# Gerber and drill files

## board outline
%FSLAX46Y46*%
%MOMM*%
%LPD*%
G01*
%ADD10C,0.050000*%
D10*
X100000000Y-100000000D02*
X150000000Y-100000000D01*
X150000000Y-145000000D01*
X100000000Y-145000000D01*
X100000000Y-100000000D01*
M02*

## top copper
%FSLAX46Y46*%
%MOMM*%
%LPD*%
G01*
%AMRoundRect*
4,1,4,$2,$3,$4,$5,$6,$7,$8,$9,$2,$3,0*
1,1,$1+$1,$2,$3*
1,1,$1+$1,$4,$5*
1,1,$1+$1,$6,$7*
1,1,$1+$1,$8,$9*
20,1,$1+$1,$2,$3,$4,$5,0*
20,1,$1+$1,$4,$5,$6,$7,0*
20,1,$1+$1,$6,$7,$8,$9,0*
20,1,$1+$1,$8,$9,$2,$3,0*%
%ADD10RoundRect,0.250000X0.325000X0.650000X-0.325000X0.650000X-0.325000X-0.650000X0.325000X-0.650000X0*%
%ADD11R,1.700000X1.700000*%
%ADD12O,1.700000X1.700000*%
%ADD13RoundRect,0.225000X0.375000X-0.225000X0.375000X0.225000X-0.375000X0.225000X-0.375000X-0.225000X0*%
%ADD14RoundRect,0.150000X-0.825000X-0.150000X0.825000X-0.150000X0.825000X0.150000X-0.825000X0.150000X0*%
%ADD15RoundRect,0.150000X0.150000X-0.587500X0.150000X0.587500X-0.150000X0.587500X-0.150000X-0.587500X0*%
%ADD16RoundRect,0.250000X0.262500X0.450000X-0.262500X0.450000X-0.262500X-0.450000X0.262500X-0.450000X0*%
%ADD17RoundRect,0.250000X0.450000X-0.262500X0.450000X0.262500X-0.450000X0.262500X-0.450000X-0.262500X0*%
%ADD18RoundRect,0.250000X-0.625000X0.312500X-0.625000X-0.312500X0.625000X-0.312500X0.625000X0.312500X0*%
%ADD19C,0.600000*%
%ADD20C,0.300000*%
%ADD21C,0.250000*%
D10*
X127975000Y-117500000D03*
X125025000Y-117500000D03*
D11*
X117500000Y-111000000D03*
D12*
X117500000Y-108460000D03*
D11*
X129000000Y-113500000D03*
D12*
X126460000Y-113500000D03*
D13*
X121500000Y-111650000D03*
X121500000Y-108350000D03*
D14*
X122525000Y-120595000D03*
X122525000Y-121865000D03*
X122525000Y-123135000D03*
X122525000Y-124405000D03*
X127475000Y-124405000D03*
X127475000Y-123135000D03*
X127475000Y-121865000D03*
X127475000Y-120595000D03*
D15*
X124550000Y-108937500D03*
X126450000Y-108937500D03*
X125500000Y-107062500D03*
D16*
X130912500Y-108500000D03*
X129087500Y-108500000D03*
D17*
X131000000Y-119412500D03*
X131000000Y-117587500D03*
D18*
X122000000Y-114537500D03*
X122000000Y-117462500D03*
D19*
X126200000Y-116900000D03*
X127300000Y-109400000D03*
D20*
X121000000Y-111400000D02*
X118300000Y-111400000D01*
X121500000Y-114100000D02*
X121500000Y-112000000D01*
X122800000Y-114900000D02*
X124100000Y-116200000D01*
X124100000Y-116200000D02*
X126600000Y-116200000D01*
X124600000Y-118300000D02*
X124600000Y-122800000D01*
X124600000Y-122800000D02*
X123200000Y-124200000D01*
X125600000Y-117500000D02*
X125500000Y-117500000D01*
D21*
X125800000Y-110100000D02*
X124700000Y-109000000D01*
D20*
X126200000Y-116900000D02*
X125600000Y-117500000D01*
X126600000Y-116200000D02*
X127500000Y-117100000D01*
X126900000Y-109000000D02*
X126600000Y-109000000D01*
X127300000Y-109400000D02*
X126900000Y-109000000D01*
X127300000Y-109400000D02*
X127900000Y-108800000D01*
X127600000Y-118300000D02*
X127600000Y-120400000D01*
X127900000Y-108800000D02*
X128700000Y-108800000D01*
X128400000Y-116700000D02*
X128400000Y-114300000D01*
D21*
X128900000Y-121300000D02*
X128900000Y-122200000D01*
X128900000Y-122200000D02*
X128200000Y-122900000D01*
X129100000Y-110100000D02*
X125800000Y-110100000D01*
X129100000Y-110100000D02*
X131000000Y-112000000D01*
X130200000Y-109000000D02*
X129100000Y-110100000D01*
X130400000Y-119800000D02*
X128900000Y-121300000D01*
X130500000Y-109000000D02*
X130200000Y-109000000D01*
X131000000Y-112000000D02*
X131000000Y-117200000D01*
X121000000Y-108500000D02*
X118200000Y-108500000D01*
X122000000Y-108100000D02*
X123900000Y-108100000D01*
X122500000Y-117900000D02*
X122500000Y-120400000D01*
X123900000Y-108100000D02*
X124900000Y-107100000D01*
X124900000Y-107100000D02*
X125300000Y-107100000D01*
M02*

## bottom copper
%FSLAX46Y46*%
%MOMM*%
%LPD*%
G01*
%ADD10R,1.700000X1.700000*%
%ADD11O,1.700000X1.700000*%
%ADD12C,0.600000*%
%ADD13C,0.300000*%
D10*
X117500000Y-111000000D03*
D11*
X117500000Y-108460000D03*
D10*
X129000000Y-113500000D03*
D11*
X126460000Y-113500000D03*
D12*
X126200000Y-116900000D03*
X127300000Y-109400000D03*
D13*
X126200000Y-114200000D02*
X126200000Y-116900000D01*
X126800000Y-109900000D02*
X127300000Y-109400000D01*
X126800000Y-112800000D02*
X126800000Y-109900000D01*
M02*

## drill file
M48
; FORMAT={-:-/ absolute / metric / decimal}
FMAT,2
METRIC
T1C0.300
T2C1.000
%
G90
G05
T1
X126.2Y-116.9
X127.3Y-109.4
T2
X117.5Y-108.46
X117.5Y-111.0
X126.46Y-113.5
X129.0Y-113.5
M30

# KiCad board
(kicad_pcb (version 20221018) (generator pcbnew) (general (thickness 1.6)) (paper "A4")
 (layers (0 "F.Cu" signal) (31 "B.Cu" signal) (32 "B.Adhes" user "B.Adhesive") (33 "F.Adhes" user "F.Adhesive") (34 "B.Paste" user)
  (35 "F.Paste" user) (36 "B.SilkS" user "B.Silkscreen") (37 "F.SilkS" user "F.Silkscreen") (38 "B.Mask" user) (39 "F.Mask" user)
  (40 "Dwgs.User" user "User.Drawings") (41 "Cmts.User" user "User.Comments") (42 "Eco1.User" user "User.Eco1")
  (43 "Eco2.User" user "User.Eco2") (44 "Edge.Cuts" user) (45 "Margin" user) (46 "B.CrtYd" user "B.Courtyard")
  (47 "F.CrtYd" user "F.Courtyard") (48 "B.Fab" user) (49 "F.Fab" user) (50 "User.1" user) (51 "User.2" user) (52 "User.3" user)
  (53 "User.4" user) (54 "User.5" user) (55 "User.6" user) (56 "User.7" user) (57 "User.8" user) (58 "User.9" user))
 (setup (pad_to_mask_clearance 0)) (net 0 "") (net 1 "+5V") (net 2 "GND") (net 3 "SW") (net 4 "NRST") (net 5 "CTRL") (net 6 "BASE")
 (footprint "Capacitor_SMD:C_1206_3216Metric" (layer "F.Cu") (at 126.5 117.5 180)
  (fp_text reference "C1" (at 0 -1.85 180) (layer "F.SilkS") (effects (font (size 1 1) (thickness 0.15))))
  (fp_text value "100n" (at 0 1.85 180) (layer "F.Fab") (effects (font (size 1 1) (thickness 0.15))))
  (pad "1" smd roundrect (at -1.475 0 180) (size 1.15 1.8) (layers "F.Cu" "F.Paste" "F.Mask") (roundrect_rratio 0.217391) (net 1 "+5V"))
  (pad "2" smd roundrect (at 1.475 0 180) (size 1.15 1.8) (layers "F.Cu" "F.Paste" "F.Mask") (roundrect_rratio 0.217391) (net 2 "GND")))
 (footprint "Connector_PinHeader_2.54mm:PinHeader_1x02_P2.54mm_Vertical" (layer "F.Cu") (at 117.5 111 180)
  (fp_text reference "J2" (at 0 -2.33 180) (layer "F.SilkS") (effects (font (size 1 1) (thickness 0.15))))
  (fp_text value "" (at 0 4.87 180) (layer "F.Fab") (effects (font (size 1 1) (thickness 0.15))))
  (pad "1" thru_hole rect (at 0 0 180) (size 1.7 1.7) (drill 1) (layers "*.Cu" "*.Mask") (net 1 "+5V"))
  (pad "2" thru_hole oval (at 0 2.54 180) (size 1.7 1.7) (drill 1) (layers "*.Cu" "*.Mask") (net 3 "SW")))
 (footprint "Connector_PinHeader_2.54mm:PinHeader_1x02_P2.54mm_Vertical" (layer "F.Cu") (at 129 113.5 -90)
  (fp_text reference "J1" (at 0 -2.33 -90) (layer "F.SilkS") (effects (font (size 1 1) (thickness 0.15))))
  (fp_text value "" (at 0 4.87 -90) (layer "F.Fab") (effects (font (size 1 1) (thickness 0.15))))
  (pad "1" thru_hole rect (at 0 0 270) (size 1.7 1.7) (drill 1) (layers "*.Cu" "*.Mask") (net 1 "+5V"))
  (pad "2" thru_hole oval (at 0 2.54 270) (size 1.7 1.7) (drill 1) (layers "*.Cu" "*.Mask") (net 2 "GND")))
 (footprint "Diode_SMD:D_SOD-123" (layer "F.Cu") (at 121.5 110 90)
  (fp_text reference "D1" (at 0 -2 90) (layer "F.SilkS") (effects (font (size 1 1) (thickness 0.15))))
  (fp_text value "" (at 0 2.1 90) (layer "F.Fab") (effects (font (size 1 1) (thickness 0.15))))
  (pad "1" smd roundrect (at -1.65 0 90) (size 0.9 1.2) (layers "F.Cu" "F.Paste" "F.Mask") (roundrect_rratio 0.25) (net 1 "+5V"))
  (pad "2" smd roundrect (at 1.65 0 90) (size 0.9 1.2) (layers "F.Cu" "F.Paste" "F.Mask") (roundrect_rratio 0.25) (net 3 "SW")))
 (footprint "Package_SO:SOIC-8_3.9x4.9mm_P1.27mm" (layer "F.Cu") (at 125 122.5)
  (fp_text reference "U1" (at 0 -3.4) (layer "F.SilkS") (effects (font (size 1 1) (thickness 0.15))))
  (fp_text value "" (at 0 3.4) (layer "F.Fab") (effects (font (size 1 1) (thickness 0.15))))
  (pad "1" smd roundrect (at -2.475 -1.905) (size 1.95 0.6) (layers "F.Cu" "F.Paste" "F.Mask") (roundrect_rratio 0.25) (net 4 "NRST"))
  (pad "2" smd roundrect (at -2.475 -0.635) (size 1.95 0.6) (layers "F.Cu" "F.Paste" "F.Mask") (roundrect_rratio 0.25))
  (pad "3" smd roundrect (at -2.475 0.635) (size 1.95 0.6) (layers "F.Cu" "F.Paste" "F.Mask") (roundrect_rratio 0.25))
  (pad "4" smd roundrect (at -2.475 1.905) (size 1.95 0.6) (layers "F.Cu" "F.Paste" "F.Mask") (roundrect_rratio 0.25) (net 2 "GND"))
  (pad "5" smd roundrect (at 2.475 1.905) (size 1.95 0.6) (layers "F.Cu" "F.Paste" "F.Mask") (roundrect_rratio 0.25))
  (pad "6" smd roundrect (at 2.475 0.635) (size 1.95 0.6) (layers "F.Cu" "F.Paste" "F.Mask") (roundrect_rratio 0.25) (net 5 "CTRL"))
  (pad "7" smd roundrect (at 2.475 -0.635) (size 1.95 0.6) (layers "F.Cu" "F.Paste" "F.Mask") (roundrect_rratio 0.25))
  (pad "8" smd roundrect (at 2.475 -1.905) (size 1.95 0.6) (layers "F.Cu" "F.Paste" "F.Mask") (roundrect_rratio 0.25) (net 1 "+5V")))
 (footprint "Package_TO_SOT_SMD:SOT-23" (layer "F.Cu") (at 125.5 108 90)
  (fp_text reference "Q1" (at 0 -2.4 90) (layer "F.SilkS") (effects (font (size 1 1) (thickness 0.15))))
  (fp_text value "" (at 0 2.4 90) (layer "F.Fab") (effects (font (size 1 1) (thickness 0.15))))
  (pad "1" smd roundrect (at -0.9375 -0.95 90) (size 1.475 0.6) (layers "F.Cu" "F.Paste" "F.Mask") (roundrect_rratio 0.25) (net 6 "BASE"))
  (pad "2" smd roundrect (at -0.9375 0.95 90) (size 1.475 0.6) (layers "F.Cu" "F.Paste" "F.Mask") (roundrect_rratio 0.25) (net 2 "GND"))
  (pad "3" smd roundrect (at 0.9375 0 90) (size 1.475 0.6) (layers "F.Cu" "F.Paste" "F.Mask") (roundrect_rratio 0.25) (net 3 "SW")))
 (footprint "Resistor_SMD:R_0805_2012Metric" (layer "F.Cu") (at 130 108.5 180)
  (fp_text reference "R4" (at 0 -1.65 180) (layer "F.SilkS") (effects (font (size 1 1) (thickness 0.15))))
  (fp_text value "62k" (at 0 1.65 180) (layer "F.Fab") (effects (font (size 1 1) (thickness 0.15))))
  (pad "1" smd roundrect (at -0.9125 0 180) (size 1.025 1.4) (layers "F.Cu" "F.Paste" "F.Mask") (roundrect_rratio 0.243902) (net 6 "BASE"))
  (pad "2" smd roundrect (at 0.9125 0 180) (size 1.025 1.4) (layers "F.Cu" "F.Paste" "F.Mask") (roundrect_rratio 0.243902) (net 2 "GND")))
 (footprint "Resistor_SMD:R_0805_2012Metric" (layer "F.Cu") (at 131 118.5 90)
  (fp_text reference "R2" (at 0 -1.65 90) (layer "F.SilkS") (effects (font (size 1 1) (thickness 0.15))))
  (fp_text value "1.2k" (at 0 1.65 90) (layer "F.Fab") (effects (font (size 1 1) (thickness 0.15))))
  (pad "1" smd roundrect (at -0.9125 0 90) (size 1.025 1.4) (layers "F.Cu" "F.Paste" "F.Mask") (roundrect_rratio 0.243902) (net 5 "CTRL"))
  (pad "2" smd roundrect (at 0.9125 0 90) (size 1.025 1.4) (layers "F.Cu" "F.Paste" "F.Mask") (roundrect_rratio 0.243902) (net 6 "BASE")))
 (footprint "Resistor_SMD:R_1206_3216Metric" (layer "F.Cu") (at 122 116 -90)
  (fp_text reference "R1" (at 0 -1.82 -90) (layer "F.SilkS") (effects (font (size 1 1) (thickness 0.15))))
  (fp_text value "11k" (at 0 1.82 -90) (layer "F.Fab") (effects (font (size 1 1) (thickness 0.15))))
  (pad "1" smd roundrect (at -1.4625 0 270) (size 1.125 1.75) (layers "F.Cu" "F.Paste" "F.Mask") (roundrect_rratio 0.222222) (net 1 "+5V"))
  (pad "2" smd roundrect (at 1.4625 0 270) (size 1.125 1.75) (layers "F.Cu" "F.Paste" "F.Mask") (roundrect_rratio 0.222222) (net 4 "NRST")))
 (gr_rect (start 100 100) (end 150 145) (stroke (width 0.05) (type default)) (fill none) (layer "Edge.Cuts"))
 (segment (start 121 111.4) (end 118.3 111.4) (width 0.3) (layer "F.Cu") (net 1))
 (segment (start 121.5 114.1) (end 121.5 112) (width 0.3) (layer "F.Cu") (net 1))
 (segment (start 122.8 114.9) (end 124.1 116.2) (width 0.3) (layer "F.Cu") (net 1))
 (segment (start 124.1 116.2) (end 126.6 116.2) (width 0.3) (layer "F.Cu") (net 1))
 (segment (start 124.6 118.3) (end 124.6 122.8) (width 0.3) (layer "F.Cu") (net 2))
 (segment (start 124.6 122.8) (end 123.2 124.2) (width 0.3) (layer "F.Cu") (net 2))
 (segment (start 125.6 117.5) (end 125.5 117.5) (width 0.3) (layer "F.Cu") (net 2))
 (segment (start 125.8 110.1) (end 124.7 109) (width 0.25) (layer "F.Cu") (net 6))
 (segment (start 126.2 116.9) (end 125.6 117.5) (width 0.3) (layer "F.Cu") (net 2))
 (segment (start 126.6 116.2) (end 127.5 117.1) (width 0.3) (layer "F.Cu") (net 1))
 (segment (start 126.9 109) (end 126.6 109) (width 0.3) (layer "F.Cu") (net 2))
 (segment (start 127.3 109.4) (end 126.9 109) (width 0.3) (layer "F.Cu") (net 2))
 (segment (start 127.3 109.4) (end 127.9 108.8) (width 0.3) (layer "F.Cu") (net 2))
 (segment (start 127.6 118.3) (end 127.6 120.4) (width 0.3) (layer "F.Cu") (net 1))
 (segment (start 127.9 108.8) (end 128.7 108.8) (width 0.3) (layer "F.Cu") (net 2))
 (segment (start 128.4 116.7) (end 128.4 114.3) (width 0.3) (layer "F.Cu") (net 1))
 (segment (start 128.9 121.3) (end 128.9 122.2) (width 0.25) (layer "F.Cu") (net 5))
 (segment (start 128.9 122.2) (end 128.2 122.9) (width 0.25) (layer "F.Cu") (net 5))
 (segment (start 129.1 110.1) (end 125.8 110.1) (width 0.25) (layer "F.Cu") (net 6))
 (segment (start 129.1 110.1) (end 131 112) (width 0.25) (layer "F.Cu") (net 6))
 (segment (start 130.2 109) (end 129.1 110.1) (width 0.25) (layer "F.Cu") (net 6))
 (segment (start 130.4 119.8) (end 128.9 121.3) (width 0.25) (layer "F.Cu") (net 5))
 (segment (start 130.5 109) (end 130.2 109) (width 0.25) (layer "F.Cu") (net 6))
 (segment (start 131 112) (end 131 117.2) (width 0.25) (layer "F.Cu") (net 6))
 (via (at 126.2 116.9) (size 0.6) (drill 0.3) (layers "F.Cu" "B.Cu") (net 2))
 (via (at 127.3 109.4) (size 0.6) (drill 0.3) (layers "F.Cu" "B.Cu") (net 2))
 (segment (start 121 108.5) (end 118.2 108.5) (width 0.25) (layer "F.Cu") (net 3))
 (segment (start 122 108.1) (end 123.9 108.1) (width 0.25) (layer "F.Cu") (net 3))
 (segment (start 122.5 117.9) (end 122.5 120.4) (width 0.25) (layer "F.Cu") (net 4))
 (segment (start 123.9 108.1) (end 124.9 107.1) (width 0.25) (layer "F.Cu") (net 3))
 (segment (start 124.9 107.1) (end 125.3 107.1) (width 0.25) (layer "F.Cu") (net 3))
 (segment (start 126.2 114.2) (end 126.2 116.9) (width 0.3) (layer "B.Cu") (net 2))
 (segment (start 126.8 109.9) (end 127.3 109.4) (width 0.3) (layer "B.Cu") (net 2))
 (segment (start 126.8 112.8) (end 126.8 109.9) (width 0.3) (layer "B.Cu") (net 2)))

